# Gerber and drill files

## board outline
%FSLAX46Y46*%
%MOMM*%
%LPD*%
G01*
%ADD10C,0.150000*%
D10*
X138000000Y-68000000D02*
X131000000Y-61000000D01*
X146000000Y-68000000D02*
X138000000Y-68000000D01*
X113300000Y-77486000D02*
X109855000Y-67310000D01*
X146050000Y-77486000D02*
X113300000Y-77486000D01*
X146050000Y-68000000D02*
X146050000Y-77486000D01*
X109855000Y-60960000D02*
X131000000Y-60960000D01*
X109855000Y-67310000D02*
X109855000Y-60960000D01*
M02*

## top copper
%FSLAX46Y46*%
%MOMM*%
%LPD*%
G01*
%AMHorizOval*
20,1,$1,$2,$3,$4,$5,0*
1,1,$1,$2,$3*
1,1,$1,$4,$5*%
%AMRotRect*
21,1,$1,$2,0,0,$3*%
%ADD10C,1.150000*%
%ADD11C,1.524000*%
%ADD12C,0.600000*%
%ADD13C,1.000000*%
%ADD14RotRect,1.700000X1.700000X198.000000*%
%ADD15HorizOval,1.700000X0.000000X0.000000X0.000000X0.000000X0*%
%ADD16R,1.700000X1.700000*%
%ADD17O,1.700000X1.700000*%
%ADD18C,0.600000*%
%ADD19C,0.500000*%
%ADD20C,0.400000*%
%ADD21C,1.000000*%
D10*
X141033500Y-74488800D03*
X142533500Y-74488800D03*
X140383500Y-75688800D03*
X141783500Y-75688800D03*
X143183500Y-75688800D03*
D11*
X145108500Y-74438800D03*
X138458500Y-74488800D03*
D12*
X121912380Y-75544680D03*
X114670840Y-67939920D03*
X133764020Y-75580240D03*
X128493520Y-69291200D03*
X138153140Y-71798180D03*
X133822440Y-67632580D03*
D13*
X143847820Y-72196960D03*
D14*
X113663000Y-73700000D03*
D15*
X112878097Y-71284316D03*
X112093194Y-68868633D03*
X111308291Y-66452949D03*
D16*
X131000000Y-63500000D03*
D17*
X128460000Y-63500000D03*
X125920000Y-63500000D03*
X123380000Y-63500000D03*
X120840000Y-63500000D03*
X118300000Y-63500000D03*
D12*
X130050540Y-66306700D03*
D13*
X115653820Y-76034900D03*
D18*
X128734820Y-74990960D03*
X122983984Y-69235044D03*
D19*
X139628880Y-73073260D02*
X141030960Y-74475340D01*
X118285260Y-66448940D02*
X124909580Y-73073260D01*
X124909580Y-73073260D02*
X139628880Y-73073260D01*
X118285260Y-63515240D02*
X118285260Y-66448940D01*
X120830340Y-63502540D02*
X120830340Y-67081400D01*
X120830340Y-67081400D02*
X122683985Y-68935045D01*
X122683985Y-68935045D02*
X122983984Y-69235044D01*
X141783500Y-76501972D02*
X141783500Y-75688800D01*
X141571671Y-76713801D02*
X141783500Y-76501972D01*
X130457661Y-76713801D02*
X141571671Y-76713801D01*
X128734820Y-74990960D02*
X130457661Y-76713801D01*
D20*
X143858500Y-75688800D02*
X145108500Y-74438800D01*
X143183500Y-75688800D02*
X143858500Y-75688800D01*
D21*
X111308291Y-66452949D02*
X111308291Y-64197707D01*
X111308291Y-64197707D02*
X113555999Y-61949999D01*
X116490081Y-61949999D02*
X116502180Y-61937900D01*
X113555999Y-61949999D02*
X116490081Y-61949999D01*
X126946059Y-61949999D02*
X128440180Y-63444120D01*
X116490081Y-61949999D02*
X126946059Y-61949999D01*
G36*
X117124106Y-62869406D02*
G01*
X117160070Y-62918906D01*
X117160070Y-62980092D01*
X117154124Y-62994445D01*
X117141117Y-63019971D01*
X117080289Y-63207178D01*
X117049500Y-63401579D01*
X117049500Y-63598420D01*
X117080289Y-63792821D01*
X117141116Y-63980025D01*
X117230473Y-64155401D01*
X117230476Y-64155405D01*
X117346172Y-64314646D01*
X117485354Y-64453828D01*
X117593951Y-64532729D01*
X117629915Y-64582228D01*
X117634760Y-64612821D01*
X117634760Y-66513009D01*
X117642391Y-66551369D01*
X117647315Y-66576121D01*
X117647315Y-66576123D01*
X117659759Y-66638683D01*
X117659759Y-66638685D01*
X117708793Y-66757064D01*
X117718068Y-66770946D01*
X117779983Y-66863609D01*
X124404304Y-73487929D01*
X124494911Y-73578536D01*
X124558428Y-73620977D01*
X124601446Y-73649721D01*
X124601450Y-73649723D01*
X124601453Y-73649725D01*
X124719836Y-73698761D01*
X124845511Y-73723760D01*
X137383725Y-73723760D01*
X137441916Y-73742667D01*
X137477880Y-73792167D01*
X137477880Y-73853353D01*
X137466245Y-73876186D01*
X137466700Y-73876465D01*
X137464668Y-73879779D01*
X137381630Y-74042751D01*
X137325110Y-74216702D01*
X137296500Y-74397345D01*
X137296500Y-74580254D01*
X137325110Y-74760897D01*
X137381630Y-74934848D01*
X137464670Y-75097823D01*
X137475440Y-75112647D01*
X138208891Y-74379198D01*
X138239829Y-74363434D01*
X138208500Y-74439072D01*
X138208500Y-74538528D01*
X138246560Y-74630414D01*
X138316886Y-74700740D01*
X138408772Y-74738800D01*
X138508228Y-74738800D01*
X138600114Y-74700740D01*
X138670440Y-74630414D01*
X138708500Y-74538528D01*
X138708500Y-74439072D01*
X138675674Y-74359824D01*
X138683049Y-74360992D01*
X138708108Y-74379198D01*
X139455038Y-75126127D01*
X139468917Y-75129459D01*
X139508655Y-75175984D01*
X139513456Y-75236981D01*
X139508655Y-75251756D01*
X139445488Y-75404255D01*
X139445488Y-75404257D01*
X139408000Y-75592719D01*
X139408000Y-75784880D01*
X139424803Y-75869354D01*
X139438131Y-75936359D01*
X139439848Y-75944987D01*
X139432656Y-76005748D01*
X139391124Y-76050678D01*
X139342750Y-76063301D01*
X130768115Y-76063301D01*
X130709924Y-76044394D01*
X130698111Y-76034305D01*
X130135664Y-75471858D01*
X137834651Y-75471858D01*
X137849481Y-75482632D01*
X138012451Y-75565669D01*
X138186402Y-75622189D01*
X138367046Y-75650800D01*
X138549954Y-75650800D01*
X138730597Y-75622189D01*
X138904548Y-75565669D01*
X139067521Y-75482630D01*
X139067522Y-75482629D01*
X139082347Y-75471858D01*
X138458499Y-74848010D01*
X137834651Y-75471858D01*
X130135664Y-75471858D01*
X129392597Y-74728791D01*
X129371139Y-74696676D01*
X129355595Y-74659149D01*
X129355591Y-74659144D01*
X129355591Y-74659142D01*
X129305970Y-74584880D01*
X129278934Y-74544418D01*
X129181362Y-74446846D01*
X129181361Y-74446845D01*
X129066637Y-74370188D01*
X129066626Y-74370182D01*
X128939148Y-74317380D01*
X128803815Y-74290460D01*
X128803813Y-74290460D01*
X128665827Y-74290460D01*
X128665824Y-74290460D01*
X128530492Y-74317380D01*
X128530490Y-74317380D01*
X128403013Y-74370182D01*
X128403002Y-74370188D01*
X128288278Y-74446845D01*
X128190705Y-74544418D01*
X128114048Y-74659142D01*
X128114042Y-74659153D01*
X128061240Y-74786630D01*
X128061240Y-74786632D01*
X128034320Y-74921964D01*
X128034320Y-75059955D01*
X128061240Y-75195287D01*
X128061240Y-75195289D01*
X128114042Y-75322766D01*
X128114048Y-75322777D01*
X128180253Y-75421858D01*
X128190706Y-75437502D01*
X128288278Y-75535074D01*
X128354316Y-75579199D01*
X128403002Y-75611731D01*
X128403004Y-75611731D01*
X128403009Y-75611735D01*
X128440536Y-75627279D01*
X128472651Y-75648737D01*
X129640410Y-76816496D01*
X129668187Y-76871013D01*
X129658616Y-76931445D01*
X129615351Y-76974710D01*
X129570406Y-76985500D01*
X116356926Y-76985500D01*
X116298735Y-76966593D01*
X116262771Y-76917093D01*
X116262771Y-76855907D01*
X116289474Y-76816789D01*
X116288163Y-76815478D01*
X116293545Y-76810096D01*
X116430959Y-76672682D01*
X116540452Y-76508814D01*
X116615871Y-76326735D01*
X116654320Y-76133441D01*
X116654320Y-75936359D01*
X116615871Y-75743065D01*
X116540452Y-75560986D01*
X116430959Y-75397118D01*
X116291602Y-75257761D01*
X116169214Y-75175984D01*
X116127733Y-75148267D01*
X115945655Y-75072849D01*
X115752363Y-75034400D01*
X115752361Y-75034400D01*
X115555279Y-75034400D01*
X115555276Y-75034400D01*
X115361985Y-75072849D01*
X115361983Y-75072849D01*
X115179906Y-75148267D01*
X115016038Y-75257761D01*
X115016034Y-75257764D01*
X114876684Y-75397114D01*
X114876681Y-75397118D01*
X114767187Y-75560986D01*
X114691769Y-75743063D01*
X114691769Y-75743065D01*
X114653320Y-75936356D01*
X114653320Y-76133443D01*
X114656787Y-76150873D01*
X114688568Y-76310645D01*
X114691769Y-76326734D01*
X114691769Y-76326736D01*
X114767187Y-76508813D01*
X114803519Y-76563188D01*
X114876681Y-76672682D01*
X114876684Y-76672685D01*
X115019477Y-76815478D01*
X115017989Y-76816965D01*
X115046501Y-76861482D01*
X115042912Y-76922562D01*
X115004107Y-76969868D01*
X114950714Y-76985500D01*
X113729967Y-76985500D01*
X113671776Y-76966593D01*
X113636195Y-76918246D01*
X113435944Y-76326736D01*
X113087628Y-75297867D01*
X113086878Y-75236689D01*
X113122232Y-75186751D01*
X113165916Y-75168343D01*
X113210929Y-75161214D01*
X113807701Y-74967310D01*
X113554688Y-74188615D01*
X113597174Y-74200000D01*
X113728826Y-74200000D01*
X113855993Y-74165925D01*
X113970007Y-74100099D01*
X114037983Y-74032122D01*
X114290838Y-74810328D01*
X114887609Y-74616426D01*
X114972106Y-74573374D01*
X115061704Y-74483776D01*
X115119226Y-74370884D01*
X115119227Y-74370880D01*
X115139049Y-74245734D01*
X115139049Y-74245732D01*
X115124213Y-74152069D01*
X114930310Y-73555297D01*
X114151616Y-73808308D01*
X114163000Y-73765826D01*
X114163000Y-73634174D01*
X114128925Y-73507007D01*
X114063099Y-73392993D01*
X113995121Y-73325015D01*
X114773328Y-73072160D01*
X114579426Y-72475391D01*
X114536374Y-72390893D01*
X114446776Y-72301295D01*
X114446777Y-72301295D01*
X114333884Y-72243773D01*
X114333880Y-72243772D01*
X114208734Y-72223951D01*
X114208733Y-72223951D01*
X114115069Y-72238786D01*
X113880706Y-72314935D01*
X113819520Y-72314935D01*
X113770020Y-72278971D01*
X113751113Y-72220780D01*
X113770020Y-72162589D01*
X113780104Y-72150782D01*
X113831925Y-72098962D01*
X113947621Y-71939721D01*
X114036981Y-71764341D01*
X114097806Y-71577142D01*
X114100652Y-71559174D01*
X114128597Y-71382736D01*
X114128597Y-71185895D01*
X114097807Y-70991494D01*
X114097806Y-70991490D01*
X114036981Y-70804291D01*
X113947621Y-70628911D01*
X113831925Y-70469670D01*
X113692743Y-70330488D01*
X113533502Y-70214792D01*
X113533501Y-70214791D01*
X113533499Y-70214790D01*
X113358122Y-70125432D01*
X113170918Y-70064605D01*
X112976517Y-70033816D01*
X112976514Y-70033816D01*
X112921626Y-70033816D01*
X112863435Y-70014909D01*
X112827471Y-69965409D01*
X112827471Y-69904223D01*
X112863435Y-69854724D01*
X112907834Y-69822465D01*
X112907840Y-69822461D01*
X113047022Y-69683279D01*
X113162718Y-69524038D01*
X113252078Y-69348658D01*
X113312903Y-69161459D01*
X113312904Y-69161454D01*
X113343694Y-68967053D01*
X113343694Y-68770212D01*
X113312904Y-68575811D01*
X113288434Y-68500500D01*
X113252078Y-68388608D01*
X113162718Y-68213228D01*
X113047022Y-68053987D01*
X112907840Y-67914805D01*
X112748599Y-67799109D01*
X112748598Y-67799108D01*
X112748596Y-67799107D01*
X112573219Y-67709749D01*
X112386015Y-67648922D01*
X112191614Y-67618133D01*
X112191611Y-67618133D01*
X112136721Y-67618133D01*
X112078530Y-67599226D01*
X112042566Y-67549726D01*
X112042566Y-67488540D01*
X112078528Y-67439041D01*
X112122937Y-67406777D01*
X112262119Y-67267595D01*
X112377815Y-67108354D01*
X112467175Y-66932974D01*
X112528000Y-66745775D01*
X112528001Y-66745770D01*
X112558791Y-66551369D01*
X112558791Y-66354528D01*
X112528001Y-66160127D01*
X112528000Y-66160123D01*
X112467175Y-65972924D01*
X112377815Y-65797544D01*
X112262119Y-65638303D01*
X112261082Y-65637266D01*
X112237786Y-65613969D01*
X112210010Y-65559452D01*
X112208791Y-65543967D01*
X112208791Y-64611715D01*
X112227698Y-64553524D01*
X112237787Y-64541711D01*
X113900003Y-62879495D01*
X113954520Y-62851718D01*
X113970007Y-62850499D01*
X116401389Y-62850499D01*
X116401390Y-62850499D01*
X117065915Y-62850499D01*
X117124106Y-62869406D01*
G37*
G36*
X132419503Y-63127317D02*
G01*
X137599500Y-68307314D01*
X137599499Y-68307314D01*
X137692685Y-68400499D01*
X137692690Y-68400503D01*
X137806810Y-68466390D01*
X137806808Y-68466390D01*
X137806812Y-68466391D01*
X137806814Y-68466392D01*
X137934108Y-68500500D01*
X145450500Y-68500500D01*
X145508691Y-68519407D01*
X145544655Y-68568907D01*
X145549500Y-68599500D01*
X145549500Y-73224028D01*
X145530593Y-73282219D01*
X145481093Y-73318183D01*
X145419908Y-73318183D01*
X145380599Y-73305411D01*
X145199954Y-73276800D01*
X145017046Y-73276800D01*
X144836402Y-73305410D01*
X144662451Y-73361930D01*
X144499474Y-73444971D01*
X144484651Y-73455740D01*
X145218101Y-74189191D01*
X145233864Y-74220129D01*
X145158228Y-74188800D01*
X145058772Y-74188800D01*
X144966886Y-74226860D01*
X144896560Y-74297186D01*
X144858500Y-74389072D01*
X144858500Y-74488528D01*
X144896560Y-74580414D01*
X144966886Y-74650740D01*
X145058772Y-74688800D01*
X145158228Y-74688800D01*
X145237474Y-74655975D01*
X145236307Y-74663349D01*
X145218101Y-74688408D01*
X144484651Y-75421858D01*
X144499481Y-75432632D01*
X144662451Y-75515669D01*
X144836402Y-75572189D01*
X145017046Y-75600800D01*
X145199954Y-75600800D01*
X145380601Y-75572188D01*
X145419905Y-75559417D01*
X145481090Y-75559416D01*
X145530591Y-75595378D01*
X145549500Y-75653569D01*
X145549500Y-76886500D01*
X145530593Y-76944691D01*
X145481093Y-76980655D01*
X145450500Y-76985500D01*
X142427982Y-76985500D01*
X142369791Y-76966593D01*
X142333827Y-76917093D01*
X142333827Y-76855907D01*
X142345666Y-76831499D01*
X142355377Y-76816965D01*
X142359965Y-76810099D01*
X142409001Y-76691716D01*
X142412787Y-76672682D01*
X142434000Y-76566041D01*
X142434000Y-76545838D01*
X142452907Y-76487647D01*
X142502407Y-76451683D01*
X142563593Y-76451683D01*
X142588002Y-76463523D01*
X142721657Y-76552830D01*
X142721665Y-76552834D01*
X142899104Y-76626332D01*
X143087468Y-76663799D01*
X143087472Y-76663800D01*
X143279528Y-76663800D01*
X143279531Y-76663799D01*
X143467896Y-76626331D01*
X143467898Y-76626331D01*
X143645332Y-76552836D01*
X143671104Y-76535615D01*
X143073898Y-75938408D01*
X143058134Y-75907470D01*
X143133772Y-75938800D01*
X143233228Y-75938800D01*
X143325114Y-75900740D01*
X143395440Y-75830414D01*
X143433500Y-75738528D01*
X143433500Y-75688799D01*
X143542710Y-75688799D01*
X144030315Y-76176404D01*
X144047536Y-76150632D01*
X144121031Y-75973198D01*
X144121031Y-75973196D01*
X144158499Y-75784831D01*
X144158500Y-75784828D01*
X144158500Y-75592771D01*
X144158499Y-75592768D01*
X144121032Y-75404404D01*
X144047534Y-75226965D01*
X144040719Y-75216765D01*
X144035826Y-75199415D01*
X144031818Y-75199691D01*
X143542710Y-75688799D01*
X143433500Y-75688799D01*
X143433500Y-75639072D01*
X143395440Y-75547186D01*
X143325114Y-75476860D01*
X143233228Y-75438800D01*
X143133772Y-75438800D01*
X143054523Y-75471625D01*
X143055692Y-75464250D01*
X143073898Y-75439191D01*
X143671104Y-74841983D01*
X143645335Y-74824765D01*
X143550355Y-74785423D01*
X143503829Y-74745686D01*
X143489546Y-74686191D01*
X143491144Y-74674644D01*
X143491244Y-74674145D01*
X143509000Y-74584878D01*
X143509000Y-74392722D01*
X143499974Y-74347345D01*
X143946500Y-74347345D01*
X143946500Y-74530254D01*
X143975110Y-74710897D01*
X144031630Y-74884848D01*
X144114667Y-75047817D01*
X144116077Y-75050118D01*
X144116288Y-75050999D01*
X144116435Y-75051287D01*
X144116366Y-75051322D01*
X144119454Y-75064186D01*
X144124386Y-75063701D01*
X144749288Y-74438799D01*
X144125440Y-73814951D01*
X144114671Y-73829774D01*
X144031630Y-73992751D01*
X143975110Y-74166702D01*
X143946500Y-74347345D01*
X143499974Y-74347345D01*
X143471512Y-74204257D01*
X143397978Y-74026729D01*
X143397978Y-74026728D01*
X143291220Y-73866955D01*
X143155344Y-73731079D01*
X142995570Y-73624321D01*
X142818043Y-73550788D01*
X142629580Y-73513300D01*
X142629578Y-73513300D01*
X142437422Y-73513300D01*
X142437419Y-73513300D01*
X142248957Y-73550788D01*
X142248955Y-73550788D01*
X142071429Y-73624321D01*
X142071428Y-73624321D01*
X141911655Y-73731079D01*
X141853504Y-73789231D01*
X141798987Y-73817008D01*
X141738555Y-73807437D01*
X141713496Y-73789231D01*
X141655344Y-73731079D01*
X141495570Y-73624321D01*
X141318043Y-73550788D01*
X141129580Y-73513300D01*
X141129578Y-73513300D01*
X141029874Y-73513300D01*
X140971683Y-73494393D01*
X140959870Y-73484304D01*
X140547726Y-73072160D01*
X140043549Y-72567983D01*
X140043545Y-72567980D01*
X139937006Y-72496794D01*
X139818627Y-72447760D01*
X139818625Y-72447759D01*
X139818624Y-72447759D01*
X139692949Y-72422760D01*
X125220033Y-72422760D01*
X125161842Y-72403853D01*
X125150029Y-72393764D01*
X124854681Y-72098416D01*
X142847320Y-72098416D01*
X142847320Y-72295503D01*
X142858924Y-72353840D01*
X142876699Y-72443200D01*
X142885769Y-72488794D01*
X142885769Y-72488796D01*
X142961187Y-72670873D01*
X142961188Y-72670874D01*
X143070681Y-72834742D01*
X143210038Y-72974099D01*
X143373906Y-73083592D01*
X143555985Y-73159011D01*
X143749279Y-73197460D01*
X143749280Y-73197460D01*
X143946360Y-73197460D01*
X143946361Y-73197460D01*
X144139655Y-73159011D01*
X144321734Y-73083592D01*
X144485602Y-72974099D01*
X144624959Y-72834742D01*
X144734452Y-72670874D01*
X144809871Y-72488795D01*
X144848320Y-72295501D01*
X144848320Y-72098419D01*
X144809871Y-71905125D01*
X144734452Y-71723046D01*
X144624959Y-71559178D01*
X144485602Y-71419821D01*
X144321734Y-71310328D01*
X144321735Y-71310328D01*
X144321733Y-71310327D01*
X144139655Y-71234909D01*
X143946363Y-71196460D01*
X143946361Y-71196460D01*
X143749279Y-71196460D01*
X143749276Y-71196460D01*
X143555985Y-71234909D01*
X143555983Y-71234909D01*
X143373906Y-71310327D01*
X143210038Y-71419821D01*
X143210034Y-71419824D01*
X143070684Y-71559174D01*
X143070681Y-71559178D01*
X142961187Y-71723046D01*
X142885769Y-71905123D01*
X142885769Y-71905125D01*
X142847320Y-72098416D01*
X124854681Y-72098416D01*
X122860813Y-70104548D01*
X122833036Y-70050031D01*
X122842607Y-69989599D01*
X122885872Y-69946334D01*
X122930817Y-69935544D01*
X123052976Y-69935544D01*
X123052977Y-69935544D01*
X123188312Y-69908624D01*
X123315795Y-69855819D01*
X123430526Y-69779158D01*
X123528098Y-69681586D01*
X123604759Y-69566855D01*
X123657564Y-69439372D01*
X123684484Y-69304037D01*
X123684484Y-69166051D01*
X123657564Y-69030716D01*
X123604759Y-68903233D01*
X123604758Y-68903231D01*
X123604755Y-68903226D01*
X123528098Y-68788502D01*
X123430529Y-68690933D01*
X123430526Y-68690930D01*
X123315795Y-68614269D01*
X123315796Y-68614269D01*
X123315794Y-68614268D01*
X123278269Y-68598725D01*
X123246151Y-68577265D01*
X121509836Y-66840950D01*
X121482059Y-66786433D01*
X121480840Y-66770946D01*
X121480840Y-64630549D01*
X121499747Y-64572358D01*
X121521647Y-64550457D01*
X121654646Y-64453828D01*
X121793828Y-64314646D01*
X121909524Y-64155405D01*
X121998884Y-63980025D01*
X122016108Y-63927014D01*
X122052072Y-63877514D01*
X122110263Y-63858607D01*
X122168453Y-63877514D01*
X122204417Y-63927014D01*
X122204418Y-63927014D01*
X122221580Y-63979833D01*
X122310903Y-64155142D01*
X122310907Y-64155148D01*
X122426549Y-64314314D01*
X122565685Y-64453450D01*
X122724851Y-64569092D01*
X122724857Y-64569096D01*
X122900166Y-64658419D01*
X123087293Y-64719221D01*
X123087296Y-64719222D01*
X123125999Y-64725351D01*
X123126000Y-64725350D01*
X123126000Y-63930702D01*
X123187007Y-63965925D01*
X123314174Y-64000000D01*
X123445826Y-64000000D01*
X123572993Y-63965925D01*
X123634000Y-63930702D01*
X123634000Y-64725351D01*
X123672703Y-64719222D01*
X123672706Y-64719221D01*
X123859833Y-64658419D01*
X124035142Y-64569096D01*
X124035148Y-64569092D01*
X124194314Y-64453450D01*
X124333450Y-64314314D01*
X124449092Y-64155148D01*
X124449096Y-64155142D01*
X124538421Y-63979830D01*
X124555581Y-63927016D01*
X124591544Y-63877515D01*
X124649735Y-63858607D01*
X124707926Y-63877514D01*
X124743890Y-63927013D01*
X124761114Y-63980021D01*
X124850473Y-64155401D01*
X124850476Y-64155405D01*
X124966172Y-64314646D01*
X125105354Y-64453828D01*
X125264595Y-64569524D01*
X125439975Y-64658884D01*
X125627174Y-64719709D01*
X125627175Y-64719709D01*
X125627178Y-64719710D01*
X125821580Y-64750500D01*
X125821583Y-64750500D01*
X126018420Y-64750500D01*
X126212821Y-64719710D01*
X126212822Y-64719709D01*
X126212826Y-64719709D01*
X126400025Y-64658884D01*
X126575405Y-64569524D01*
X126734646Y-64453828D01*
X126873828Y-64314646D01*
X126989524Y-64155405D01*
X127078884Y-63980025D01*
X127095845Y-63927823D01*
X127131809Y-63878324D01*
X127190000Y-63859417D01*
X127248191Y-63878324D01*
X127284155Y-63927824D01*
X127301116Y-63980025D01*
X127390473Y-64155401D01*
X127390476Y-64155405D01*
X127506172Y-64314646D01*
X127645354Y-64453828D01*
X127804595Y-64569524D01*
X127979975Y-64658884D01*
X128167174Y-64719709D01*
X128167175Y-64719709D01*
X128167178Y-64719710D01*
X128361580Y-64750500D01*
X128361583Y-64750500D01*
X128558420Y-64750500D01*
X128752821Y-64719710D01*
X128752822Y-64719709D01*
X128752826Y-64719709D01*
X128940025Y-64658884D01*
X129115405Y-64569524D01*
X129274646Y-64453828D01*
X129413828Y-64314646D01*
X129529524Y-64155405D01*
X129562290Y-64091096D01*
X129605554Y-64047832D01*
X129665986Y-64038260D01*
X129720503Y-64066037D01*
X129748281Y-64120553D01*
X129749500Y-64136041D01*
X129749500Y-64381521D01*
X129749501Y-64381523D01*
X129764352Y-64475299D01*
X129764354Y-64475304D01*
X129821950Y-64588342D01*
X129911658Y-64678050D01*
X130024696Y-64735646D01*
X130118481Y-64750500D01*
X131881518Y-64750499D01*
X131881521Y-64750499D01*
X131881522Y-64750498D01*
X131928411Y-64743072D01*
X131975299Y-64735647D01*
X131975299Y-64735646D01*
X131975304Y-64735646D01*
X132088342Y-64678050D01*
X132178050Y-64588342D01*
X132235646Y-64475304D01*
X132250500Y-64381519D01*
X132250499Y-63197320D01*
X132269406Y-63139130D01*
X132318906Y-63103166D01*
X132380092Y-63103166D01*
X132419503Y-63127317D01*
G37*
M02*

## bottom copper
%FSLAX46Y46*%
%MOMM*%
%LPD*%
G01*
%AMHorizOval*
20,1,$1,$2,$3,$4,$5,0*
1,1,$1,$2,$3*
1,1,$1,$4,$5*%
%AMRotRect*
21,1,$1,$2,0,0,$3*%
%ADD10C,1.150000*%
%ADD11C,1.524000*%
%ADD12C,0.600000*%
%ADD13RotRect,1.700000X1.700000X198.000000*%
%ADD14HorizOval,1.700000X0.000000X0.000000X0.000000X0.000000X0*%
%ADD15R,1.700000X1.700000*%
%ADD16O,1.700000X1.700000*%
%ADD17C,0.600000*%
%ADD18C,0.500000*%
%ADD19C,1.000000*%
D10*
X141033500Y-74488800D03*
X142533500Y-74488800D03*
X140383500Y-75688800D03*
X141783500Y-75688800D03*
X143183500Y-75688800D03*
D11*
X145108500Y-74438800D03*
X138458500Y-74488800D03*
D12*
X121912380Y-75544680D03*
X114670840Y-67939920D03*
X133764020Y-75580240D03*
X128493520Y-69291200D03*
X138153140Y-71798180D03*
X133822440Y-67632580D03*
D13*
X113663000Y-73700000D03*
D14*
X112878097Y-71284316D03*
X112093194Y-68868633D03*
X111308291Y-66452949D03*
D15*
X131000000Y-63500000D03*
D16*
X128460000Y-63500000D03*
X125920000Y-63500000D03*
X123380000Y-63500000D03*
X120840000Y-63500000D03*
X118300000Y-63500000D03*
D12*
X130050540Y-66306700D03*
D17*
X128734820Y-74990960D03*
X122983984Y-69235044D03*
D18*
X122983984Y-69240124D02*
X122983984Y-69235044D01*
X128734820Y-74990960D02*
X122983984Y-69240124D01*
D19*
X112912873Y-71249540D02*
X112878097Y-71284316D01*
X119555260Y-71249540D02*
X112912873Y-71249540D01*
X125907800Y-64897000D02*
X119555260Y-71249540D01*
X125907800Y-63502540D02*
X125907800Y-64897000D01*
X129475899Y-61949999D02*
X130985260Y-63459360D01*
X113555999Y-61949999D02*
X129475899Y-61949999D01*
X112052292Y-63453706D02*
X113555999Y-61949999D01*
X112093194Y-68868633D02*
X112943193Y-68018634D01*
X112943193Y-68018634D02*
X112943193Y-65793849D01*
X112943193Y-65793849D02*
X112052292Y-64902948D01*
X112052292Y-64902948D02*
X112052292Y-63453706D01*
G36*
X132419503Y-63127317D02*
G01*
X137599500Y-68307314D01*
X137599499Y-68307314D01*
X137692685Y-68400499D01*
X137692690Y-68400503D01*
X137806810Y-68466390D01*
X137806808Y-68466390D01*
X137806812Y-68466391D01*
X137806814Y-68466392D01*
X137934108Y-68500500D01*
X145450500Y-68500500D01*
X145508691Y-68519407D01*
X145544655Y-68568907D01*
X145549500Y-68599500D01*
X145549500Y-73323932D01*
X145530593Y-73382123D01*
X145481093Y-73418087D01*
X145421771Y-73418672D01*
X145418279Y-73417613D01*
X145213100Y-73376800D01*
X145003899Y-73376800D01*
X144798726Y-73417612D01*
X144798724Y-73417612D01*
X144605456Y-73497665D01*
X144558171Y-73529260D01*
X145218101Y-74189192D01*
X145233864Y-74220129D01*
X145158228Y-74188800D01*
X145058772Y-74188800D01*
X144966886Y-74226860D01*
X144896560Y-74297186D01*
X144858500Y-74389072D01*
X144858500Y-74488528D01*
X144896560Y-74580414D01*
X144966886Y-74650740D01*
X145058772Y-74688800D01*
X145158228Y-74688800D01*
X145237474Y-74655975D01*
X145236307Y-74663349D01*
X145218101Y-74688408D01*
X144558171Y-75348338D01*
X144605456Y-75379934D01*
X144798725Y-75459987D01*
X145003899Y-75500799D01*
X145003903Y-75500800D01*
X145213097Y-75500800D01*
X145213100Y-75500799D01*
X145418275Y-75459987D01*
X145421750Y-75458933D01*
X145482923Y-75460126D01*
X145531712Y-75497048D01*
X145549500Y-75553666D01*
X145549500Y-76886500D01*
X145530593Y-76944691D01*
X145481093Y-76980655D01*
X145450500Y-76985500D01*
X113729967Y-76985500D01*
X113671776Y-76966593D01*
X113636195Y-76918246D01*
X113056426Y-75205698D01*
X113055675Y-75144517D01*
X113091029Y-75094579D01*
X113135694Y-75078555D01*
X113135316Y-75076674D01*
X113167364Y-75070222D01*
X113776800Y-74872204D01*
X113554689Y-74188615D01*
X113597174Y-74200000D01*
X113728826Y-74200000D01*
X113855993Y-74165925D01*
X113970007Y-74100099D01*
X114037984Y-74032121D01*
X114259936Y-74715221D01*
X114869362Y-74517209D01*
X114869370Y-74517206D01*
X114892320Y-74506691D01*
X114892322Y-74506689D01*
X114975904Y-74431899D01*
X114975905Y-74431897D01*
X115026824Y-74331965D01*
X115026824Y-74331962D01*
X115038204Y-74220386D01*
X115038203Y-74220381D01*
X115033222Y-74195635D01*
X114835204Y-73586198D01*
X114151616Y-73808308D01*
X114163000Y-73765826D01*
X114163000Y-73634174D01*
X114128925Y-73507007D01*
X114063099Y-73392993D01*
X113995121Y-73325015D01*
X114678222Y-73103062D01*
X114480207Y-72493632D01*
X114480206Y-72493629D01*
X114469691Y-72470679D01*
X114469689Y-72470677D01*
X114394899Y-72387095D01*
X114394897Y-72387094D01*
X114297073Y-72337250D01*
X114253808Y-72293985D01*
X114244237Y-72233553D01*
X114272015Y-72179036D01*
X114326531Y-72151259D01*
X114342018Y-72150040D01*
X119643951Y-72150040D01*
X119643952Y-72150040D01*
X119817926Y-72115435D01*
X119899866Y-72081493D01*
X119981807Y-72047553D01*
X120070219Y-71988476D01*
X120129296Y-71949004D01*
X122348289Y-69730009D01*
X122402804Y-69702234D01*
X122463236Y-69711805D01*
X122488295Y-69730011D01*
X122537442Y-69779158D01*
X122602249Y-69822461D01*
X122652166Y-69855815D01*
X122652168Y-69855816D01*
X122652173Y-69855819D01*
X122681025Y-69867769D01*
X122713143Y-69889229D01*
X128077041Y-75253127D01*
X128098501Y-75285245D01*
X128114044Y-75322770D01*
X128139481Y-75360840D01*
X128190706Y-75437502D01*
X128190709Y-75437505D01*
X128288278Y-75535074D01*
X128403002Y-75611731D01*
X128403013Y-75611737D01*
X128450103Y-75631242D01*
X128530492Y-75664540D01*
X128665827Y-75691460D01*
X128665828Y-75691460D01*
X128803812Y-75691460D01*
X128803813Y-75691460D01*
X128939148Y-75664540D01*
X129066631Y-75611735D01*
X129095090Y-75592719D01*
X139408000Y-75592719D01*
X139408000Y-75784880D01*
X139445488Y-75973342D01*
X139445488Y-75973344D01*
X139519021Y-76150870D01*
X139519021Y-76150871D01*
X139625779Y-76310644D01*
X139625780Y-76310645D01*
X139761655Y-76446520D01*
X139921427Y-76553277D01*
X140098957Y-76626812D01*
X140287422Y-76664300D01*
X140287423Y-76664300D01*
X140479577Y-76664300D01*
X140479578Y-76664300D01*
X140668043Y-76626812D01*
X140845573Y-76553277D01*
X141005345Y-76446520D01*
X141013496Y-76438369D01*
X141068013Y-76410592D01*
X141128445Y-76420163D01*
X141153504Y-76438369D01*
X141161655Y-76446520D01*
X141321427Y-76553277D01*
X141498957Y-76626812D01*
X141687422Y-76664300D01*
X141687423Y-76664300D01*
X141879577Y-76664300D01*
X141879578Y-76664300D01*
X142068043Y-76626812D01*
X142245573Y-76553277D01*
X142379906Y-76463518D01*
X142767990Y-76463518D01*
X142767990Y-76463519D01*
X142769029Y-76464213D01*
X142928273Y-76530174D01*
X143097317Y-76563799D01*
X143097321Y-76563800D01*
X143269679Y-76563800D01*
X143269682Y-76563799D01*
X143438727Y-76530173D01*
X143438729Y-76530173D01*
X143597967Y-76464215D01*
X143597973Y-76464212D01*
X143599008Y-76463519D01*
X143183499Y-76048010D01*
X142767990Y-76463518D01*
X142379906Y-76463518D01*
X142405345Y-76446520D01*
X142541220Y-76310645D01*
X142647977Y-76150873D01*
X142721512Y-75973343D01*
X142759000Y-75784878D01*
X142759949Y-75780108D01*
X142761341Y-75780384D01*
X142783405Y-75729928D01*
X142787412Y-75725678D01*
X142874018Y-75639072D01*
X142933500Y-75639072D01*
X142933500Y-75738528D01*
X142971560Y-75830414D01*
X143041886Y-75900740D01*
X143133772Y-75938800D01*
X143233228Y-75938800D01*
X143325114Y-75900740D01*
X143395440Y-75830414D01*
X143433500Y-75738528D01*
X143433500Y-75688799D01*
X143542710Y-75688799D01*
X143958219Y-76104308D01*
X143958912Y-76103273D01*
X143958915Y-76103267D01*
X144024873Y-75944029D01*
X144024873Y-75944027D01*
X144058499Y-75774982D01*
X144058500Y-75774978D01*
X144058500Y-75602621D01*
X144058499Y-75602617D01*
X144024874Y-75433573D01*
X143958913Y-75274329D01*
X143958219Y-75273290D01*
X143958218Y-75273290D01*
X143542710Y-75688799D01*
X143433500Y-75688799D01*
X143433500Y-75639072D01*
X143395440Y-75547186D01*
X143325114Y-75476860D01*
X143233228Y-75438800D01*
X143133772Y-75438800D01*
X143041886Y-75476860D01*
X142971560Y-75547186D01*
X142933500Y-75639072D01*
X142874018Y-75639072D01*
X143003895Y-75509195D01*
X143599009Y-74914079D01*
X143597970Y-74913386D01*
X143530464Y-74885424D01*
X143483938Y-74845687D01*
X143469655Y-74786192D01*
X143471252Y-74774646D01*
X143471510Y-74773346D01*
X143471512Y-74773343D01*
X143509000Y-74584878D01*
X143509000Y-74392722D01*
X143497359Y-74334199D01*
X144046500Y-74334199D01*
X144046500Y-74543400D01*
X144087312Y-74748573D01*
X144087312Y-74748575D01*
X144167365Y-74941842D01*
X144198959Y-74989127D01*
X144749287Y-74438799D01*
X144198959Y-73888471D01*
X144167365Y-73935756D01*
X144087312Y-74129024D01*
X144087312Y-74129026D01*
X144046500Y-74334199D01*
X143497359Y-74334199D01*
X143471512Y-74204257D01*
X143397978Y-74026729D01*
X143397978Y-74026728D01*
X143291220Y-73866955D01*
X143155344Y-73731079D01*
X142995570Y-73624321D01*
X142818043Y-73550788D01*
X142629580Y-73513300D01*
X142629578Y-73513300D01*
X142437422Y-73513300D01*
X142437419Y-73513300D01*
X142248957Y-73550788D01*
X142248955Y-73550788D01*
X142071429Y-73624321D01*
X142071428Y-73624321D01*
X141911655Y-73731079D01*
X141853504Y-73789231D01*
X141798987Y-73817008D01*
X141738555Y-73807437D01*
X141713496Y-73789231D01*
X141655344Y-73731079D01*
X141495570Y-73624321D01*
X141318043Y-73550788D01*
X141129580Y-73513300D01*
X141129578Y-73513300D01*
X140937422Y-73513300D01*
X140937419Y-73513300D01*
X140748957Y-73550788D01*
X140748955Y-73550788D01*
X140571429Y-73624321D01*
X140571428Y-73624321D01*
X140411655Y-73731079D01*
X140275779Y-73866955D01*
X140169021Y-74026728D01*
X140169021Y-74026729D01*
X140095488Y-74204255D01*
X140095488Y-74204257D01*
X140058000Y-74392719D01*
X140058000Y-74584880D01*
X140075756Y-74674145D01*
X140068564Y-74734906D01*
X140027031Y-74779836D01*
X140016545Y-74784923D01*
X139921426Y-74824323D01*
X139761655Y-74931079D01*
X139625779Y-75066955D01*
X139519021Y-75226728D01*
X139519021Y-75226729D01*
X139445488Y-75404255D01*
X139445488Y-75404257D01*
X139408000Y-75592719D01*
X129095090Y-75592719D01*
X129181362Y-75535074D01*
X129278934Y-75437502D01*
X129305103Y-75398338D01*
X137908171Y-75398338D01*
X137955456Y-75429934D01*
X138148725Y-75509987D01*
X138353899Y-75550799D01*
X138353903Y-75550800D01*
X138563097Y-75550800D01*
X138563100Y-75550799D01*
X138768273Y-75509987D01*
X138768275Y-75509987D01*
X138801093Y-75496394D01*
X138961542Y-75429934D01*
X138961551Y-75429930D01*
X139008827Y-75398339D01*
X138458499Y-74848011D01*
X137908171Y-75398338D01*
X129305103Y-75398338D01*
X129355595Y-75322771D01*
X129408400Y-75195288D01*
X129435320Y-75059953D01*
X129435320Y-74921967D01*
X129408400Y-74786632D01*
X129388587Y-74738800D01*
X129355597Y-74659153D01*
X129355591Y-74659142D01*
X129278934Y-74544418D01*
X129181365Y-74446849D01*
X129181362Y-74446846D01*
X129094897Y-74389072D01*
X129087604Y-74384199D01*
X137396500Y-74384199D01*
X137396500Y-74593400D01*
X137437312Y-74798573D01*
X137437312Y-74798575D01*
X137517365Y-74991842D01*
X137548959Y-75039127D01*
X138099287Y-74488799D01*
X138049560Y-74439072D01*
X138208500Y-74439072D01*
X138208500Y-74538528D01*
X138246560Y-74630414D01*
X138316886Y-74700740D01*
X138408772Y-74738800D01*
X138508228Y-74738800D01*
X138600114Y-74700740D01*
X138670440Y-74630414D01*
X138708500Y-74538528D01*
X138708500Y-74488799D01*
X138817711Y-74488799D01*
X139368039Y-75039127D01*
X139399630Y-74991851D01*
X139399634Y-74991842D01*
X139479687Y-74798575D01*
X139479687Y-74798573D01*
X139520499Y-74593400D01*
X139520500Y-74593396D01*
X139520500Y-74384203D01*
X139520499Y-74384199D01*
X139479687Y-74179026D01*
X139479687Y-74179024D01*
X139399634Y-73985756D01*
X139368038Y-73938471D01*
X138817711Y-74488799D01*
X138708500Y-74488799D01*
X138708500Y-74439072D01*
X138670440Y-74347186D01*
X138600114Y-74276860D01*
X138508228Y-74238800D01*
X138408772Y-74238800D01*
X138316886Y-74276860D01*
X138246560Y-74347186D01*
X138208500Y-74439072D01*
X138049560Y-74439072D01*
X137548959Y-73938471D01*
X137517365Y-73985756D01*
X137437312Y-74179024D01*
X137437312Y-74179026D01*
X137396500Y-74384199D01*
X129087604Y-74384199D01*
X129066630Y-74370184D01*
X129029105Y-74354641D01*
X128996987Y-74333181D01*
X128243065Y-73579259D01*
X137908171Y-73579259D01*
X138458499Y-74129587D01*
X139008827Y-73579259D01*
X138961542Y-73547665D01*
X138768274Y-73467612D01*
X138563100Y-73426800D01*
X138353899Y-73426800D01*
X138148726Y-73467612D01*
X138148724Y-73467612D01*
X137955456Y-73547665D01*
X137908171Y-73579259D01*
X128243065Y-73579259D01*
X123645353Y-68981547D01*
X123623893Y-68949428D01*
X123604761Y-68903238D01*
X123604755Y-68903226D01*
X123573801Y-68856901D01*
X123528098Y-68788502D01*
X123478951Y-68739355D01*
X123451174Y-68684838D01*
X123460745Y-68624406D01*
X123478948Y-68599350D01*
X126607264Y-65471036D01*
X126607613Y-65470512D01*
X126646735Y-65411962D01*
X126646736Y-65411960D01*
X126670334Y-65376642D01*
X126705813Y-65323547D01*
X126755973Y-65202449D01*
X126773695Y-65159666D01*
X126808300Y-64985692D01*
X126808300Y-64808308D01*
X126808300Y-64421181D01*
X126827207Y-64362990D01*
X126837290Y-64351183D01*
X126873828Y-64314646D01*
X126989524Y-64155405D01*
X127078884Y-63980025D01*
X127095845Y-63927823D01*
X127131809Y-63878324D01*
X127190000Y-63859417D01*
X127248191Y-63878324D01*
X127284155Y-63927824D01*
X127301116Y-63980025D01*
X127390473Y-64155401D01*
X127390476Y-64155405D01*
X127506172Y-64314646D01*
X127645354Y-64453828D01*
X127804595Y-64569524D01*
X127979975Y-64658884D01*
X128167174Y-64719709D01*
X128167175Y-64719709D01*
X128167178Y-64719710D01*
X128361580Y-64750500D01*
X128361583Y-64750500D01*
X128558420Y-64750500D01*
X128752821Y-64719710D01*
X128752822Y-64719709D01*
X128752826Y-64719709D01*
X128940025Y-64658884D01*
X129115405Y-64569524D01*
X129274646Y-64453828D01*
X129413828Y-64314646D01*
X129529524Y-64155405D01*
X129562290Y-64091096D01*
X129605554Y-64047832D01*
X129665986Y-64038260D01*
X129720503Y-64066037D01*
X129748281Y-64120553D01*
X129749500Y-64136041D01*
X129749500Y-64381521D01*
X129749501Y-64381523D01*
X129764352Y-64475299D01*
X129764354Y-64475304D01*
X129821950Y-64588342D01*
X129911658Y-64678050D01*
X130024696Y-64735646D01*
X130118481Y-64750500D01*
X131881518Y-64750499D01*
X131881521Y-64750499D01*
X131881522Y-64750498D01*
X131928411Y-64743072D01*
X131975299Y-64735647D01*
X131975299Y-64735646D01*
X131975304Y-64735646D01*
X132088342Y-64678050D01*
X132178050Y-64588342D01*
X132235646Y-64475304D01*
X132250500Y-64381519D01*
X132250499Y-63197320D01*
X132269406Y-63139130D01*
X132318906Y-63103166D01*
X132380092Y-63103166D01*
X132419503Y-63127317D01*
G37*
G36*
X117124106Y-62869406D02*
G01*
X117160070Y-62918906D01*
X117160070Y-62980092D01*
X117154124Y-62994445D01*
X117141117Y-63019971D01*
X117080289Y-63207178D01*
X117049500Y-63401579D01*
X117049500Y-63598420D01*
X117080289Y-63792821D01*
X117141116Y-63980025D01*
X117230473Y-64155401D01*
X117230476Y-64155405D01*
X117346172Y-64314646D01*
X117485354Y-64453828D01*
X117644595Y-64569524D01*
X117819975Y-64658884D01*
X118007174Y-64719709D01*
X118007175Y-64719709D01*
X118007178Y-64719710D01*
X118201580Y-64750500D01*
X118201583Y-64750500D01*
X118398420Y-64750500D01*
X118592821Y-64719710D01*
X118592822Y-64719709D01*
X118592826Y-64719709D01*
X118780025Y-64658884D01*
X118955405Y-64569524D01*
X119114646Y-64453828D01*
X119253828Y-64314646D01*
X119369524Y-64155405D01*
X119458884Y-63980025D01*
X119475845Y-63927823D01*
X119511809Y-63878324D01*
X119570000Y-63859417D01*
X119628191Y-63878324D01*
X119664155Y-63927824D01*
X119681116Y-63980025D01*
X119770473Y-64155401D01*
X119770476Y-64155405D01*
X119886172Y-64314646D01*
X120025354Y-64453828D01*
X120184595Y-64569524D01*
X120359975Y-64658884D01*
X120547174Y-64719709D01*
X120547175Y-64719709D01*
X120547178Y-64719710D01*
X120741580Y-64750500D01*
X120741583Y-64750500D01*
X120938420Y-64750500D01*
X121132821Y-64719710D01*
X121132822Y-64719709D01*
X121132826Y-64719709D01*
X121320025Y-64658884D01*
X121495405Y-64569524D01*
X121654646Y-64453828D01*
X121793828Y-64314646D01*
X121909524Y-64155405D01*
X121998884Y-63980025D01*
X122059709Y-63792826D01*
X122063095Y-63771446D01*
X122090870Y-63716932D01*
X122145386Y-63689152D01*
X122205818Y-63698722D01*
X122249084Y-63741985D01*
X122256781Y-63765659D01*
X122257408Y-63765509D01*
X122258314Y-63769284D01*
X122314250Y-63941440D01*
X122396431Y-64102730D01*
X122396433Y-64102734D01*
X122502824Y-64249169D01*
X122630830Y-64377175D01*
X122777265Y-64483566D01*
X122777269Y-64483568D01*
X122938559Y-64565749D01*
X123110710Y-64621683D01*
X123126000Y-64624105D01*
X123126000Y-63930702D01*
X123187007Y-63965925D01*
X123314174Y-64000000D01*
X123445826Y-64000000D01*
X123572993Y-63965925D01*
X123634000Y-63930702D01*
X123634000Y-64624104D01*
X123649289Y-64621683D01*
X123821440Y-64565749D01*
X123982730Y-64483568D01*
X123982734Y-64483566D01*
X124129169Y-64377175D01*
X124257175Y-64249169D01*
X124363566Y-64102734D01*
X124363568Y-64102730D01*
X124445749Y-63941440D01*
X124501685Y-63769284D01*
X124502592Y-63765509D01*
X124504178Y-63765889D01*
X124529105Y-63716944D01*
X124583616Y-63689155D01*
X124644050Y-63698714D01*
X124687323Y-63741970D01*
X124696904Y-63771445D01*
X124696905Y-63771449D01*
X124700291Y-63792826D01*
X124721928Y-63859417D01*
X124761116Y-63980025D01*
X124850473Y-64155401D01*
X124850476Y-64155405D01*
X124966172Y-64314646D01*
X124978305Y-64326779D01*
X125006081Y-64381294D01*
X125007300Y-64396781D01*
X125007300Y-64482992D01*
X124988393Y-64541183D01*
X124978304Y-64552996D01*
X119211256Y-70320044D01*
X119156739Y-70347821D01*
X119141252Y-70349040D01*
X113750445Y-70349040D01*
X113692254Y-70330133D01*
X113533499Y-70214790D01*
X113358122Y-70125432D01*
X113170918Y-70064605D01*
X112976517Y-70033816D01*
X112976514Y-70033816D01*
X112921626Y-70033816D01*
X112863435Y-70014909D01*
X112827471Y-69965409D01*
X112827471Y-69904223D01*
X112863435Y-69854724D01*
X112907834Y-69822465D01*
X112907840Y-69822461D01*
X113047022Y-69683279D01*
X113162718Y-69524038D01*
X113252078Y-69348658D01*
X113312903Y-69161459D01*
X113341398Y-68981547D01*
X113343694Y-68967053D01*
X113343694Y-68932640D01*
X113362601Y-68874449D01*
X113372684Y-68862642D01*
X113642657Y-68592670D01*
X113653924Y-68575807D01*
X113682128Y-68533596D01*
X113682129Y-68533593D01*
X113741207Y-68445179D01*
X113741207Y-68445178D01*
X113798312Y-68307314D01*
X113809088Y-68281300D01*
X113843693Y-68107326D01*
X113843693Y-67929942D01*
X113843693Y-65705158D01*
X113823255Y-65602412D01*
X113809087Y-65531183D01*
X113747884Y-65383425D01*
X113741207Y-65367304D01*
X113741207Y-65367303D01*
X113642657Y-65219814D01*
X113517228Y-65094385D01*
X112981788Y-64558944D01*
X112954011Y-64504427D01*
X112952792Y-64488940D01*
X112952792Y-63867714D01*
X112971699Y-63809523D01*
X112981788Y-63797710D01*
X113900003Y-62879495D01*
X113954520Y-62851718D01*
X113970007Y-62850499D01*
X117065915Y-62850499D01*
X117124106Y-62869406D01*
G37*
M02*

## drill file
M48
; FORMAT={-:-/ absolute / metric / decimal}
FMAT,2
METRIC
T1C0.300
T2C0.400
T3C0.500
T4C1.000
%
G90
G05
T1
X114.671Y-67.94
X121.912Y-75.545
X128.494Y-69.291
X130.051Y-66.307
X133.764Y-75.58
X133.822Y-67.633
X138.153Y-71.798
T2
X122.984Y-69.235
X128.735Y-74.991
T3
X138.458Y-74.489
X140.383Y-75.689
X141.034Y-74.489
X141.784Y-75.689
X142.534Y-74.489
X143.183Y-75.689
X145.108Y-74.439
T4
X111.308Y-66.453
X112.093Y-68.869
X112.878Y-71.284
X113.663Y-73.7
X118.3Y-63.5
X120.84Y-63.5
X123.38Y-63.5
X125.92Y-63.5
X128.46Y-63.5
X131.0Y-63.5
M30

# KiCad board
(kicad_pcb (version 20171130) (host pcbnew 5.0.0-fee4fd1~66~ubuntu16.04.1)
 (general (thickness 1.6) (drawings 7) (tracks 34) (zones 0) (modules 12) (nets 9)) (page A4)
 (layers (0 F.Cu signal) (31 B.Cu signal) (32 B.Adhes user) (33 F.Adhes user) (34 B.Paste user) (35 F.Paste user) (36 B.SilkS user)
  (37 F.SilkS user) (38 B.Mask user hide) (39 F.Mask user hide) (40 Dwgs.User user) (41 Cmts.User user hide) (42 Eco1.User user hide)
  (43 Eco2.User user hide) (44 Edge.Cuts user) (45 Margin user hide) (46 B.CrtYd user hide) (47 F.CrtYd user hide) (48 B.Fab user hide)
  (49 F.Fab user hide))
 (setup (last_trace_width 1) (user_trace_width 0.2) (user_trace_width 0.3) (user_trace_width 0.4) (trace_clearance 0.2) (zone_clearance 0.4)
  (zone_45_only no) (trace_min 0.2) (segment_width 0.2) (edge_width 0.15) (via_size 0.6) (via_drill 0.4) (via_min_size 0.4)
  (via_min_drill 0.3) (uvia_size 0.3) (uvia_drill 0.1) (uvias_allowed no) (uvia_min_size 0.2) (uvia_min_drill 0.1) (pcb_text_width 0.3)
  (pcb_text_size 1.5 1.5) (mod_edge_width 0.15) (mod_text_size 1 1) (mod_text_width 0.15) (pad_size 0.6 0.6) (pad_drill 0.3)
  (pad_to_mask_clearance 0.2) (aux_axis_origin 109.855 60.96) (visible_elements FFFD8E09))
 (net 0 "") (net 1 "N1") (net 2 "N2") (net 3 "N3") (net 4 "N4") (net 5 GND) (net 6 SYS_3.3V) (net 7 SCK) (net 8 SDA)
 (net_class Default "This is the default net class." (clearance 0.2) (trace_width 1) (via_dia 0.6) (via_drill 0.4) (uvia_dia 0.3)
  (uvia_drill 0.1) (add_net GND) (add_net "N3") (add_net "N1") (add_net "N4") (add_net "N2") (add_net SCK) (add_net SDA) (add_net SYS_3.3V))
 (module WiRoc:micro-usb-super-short (layer B.Cu) (at 141.7835 74.4888)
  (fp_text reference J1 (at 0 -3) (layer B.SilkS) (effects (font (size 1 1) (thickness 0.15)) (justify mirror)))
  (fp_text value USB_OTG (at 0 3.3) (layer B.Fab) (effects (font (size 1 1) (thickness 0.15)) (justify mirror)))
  (pad 2 thru_hole circle (at -0.75 0) (size 1.15 1.15) (drill 0.5) (layers *.Cu *.Mask) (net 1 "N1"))
  (pad 4 thru_hole circle (at 0.75 0) (size 1.15 1.15) (drill 0.5) (layers *.Cu *.Mask) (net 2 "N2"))
  (pad 1 thru_hole circle (at -1.4 1.2) (size 1.15 1.15) (drill 0.5) (layers *.Cu *.Mask) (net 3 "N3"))
  (pad 3 thru_hole circle (at 0 1.2) (size 1.15 1.15) (drill 0.5) (layers *.Cu *.Mask) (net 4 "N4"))
  (pad 5 thru_hole circle (at 1.4 1.2) (size 1.15 1.15) (drill 0.5) (layers *.Cu *.Mask) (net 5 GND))
  (pad 6 thru_hole circle (at 3.325 -0.05) (size 1.524 1.524) (drill 0.5) (layers *.Cu *.Mask) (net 5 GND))
  (pad 6 thru_hole circle (at -3.325 0) (size 1.524 1.524) (drill 0.5) (layers *.Cu *.Mask) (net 5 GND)))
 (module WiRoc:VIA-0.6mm (layer F.Cu) (at 121.91238 75.54468)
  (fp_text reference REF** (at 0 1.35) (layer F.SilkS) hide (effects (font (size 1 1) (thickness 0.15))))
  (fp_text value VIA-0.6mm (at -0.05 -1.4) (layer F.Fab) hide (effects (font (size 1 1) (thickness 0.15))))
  (pad 1 thru_hole circle (at 0 0) (size 0.6 0.6) (drill 0.3) (layers *.Cu) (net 5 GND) (zone_connect 2)))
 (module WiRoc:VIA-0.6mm (layer F.Cu) (at 114.67084 67.93992)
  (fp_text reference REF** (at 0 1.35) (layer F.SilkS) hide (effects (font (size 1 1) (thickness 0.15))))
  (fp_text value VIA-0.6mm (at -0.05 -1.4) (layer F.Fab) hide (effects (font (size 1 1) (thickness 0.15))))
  (pad 1 thru_hole circle (at 0 0) (size 0.6 0.6) (drill 0.3) (layers *.Cu) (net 5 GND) (zone_connect 2)))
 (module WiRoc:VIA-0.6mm (layer F.Cu) (at 133.76402 75.58024)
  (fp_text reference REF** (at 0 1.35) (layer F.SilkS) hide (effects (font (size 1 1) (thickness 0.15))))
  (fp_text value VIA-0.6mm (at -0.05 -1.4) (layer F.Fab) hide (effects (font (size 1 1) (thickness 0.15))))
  (pad 1 thru_hole circle (at 0 0) (size 0.6 0.6) (drill 0.3) (layers *.Cu) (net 5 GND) (zone_connect 2)))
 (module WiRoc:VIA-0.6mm (layer F.Cu) (at 128.49352 69.2912)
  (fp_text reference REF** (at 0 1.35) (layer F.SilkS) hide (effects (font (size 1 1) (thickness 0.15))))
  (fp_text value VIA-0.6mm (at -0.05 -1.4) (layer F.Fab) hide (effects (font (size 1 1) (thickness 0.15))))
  (pad 1 thru_hole circle (at 0 0) (size 0.6 0.6) (drill 0.3) (layers *.Cu) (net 5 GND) (zone_connect 2)))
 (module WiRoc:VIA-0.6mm (layer F.Cu) (at 138.15314 71.79818)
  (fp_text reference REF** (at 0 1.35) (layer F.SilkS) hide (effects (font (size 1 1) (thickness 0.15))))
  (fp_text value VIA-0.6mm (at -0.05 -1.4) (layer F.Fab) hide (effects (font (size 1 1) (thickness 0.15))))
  (pad 1 thru_hole circle (at 0 0) (size 0.6 0.6) (drill 0.3) (layers *.Cu) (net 5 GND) (zone_connect 2)))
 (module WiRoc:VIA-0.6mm (layer F.Cu) (at 133.82244 67.63258)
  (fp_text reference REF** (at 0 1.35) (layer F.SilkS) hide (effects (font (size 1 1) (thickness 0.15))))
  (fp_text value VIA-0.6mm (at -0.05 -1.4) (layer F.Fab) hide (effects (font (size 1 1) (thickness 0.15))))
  (pad 1 thru_hole circle (at 0 0) (size 0.6 0.6) (drill 0.3) (layers *.Cu) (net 5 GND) (zone_connect 2)))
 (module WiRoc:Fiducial (layer F.Cu) (at 143.84782 72.19696)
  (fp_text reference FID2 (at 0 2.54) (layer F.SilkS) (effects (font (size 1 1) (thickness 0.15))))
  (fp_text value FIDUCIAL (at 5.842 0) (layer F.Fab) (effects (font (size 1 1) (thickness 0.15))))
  (pad 1 smd circle (at 0 0) (size 1 1) (layers F.Cu F.Mask) (solder_mask_margin 0.5) (clearance 0.5)))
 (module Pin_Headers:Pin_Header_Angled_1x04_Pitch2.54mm (layer F.Cu) (at 113.663 73.7 198)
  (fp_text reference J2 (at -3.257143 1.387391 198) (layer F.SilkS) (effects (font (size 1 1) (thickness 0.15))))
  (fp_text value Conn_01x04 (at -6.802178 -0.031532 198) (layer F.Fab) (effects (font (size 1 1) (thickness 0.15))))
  (pad 1 thru_hole rect (at 0 0 198) (size 1.7 1.7) (drill 1) (layers *.Cu *.Mask) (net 5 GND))
  (pad 2 thru_hole oval (at 0 2.54 198) (size 1.7 1.7) (drill 1) (layers *.Cu *.Mask) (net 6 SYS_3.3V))
  (pad 3 thru_hole oval (at 0 5.08 198) (size 1.7 1.7) (drill 1) (layers *.Cu *.Mask) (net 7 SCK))
  (pad 4 thru_hole oval (at -0.000001 7.62 198) (size 1.7 1.7) (drill 1) (layers *.Cu *.Mask) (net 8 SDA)))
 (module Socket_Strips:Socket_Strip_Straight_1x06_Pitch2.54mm (layer F.Cu) (at 131 63.5 270)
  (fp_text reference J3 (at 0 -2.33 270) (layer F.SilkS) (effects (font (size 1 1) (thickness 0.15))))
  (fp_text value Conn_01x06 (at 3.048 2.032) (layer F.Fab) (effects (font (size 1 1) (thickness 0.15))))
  (pad 1 thru_hole rect (at 0 0 270) (size 1.7 1.7) (drill 1) (layers *.Cu *.Mask) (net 7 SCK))
  (pad 2 thru_hole oval (at 0 2.54 270) (size 1.7 1.7) (drill 1) (layers *.Cu *.Mask) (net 8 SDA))
  (pad 3 thru_hole oval (at 0 5.08 270) (size 1.7 1.7) (drill 1) (layers *.Cu *.Mask) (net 6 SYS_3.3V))
  (pad 4 thru_hole oval (at 0 7.62 270) (size 1.7 1.7) (drill 1) (layers *.Cu *.Mask) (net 5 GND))
  (pad 5 thru_hole oval (at 0 10.16 270) (size 1.7 1.7) (drill 1) (layers *.Cu *.Mask) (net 4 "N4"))
  (pad 6 thru_hole oval (at 0 12.7 270) (size 1.7 1.7) (drill 1) (layers *.Cu *.Mask) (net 1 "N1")))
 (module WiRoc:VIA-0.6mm (layer F.Cu) (at 130.05054 66.3067)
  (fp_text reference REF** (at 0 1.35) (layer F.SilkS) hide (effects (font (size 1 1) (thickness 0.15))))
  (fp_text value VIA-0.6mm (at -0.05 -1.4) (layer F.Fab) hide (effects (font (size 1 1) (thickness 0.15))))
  (pad 1 thru_hole circle (at 0 0) (size 0.6 0.6) (drill 0.3) (layers *.Cu) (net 5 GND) (zone_connect 2)))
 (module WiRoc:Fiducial (layer F.Cu) (at 115.65382 76.0349)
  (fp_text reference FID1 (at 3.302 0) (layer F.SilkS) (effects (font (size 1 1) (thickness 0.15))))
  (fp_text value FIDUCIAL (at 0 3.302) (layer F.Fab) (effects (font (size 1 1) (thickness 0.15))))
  (pad 1 smd circle (at 0 0) (size 1 1) (layers F.Cu F.Mask) (solder_mask_margin 0.5) (clearance 0.5)))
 (gr_line (start 138 68) (end 131 61) (layer Edge.Cuts) (width 0.15))
 (gr_line (start 146 68) (end 138 68) (layer Edge.Cuts) (width 0.15))
 (gr_line (start 113.3 77.486) (end 109.855 67.31) (layer Edge.Cuts) (width 0.15))
 (gr_line (start 146.05 77.486) (end 113.3 77.486) (layer Edge.Cuts) (width 0.15))
 (gr_line (start 146.05 68) (end 146.05 77.486) (layer Edge.Cuts) (width 0.15))
 (gr_line (start 109.855 60.96) (end 131 60.96) (layer Edge.Cuts) (width 0.15))
 (gr_line (start 109.855 67.31) (end 109.855 60.96) (layer Edge.Cuts) (width 0.15))
 (segment (start 139.62888 73.07326) (end 141.03096 74.47534) (width 0.5) (layer F.Cu) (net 1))
 (segment (start 118.28526 66.44894) (end 124.90958 73.07326) (width 0.5) (layer F.Cu) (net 1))
 (segment (start 124.90958 73.07326) (end 139.62888 73.07326) (width 0.5) (layer F.Cu) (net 1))
 (segment (start 118.28526 63.51524) (end 118.28526 66.44894) (width 0.5) (layer F.Cu) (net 1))
 (via (at 128.73482 74.99096) (size 0.6) (drill 0.4) (layers F.Cu B.Cu) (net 4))
 (segment (start 120.83034 63.50254) (end 120.83034 67.0814) (width 0.5) (layer F.Cu) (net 4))
 (segment (start 120.83034 67.0814) (end 122.683985 68.935045) (width 0.5) (layer F.Cu) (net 4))
 (segment (start 122.683985 68.935045) (end 122.983984 69.235044) (width 0.5) (layer F.Cu) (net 4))
 (segment (start 122.983984 69.240124) (end 122.983984 69.235044) (width 0.5) (layer B.Cu) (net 4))
 (segment (start 128.73482 74.99096) (end 122.983984 69.240124) (width 0.5) (layer B.Cu) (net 4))
 (via (at 122.983984 69.235044) (size 0.6) (drill 0.4) (layers F.Cu B.Cu) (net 4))
 (segment (start 141.7835 76.501972) (end 141.7835 75.6888) (width 0.5) (layer F.Cu) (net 4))
 (segment (start 141.571671 76.713801) (end 141.7835 76.501972) (width 0.5) (layer F.Cu) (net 4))
 (segment (start 130.457661 76.713801) (end 141.571671 76.713801) (width 0.5) (layer F.Cu) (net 4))
 (segment (start 128.73482 74.99096) (end 130.457661 76.713801) (width 0.5) (layer F.Cu) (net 4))
 (segment (start 143.8585 75.6888) (end 145.1085 74.4388) (width 0.4) (layer F.Cu) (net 5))
 (segment (start 143.1835 75.6888) (end 143.8585 75.6888) (width 0.4) (layer F.Cu) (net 5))
 (segment (start 112.912873 71.24954) (end 112.878097 71.284316) (width 1) (layer B.Cu) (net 6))
 (segment (start 119.55526 71.24954) (end 112.912873 71.24954) (width 1) (layer B.Cu) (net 6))
 (segment (start 125.9078 64.897) (end 119.55526 71.24954) (width 1) (layer B.Cu) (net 6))
 (segment (start 125.9078 63.50254) (end 125.9078 64.897) (width 1) (layer B.Cu) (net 6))
 (segment (start 129.475899 61.949999) (end 130.98526 63.45936) (width 1) (layer B.Cu) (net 7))
 (segment (start 113.555999 61.949999) (end 129.475899 61.949999) (width 1) (layer B.Cu) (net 7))
 (segment (start 112.052292 63.453706) (end 113.555999 61.949999) (width 1) (layer B.Cu) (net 7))
 (segment (start 112.093194 68.868633) (end 112.943193 68.018634) (width 1) (layer B.Cu) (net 7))
 (segment (start 112.943193 68.018634) (end 112.943193 65.793849) (width 1) (layer B.Cu) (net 7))
 (segment (start 112.943193 65.793849) (end 112.052292 64.902948) (width 1) (layer B.Cu) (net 7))
 (segment (start 112.052292 64.902948) (end 112.052292 63.453706) (width 1) (layer B.Cu) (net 7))
 (segment (start 111.308291 66.452949) (end 111.308291 64.197707) (width 1) (layer F.Cu) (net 8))
 (segment (start 111.308291 64.197707) (end 113.555999 61.949999) (width 1) (layer F.Cu) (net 8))
 (segment (start 116.490081 61.949999) (end 116.50218 61.9379) (width 1) (layer F.Cu) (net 8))
 (segment (start 113.555999 61.949999) (end 116.490081 61.949999) (width 1) (layer F.Cu) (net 8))
 (segment (start 126.946059 61.949999) (end 128.44018 63.44412) (width 1) (layer F.Cu) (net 8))
 (segment (start 116.490081 61.949999) (end 126.946059 61.949999) (width 1) (layer F.Cu) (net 8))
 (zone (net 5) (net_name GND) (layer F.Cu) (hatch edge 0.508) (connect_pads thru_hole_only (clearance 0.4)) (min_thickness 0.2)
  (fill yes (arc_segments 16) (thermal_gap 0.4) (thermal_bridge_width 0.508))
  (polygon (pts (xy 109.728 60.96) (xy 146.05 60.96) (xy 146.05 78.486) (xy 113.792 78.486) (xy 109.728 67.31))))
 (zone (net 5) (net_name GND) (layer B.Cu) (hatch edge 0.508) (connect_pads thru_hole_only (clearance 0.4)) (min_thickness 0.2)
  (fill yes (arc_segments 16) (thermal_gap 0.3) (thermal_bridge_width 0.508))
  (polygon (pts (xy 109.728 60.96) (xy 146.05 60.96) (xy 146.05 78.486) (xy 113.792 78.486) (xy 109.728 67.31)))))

